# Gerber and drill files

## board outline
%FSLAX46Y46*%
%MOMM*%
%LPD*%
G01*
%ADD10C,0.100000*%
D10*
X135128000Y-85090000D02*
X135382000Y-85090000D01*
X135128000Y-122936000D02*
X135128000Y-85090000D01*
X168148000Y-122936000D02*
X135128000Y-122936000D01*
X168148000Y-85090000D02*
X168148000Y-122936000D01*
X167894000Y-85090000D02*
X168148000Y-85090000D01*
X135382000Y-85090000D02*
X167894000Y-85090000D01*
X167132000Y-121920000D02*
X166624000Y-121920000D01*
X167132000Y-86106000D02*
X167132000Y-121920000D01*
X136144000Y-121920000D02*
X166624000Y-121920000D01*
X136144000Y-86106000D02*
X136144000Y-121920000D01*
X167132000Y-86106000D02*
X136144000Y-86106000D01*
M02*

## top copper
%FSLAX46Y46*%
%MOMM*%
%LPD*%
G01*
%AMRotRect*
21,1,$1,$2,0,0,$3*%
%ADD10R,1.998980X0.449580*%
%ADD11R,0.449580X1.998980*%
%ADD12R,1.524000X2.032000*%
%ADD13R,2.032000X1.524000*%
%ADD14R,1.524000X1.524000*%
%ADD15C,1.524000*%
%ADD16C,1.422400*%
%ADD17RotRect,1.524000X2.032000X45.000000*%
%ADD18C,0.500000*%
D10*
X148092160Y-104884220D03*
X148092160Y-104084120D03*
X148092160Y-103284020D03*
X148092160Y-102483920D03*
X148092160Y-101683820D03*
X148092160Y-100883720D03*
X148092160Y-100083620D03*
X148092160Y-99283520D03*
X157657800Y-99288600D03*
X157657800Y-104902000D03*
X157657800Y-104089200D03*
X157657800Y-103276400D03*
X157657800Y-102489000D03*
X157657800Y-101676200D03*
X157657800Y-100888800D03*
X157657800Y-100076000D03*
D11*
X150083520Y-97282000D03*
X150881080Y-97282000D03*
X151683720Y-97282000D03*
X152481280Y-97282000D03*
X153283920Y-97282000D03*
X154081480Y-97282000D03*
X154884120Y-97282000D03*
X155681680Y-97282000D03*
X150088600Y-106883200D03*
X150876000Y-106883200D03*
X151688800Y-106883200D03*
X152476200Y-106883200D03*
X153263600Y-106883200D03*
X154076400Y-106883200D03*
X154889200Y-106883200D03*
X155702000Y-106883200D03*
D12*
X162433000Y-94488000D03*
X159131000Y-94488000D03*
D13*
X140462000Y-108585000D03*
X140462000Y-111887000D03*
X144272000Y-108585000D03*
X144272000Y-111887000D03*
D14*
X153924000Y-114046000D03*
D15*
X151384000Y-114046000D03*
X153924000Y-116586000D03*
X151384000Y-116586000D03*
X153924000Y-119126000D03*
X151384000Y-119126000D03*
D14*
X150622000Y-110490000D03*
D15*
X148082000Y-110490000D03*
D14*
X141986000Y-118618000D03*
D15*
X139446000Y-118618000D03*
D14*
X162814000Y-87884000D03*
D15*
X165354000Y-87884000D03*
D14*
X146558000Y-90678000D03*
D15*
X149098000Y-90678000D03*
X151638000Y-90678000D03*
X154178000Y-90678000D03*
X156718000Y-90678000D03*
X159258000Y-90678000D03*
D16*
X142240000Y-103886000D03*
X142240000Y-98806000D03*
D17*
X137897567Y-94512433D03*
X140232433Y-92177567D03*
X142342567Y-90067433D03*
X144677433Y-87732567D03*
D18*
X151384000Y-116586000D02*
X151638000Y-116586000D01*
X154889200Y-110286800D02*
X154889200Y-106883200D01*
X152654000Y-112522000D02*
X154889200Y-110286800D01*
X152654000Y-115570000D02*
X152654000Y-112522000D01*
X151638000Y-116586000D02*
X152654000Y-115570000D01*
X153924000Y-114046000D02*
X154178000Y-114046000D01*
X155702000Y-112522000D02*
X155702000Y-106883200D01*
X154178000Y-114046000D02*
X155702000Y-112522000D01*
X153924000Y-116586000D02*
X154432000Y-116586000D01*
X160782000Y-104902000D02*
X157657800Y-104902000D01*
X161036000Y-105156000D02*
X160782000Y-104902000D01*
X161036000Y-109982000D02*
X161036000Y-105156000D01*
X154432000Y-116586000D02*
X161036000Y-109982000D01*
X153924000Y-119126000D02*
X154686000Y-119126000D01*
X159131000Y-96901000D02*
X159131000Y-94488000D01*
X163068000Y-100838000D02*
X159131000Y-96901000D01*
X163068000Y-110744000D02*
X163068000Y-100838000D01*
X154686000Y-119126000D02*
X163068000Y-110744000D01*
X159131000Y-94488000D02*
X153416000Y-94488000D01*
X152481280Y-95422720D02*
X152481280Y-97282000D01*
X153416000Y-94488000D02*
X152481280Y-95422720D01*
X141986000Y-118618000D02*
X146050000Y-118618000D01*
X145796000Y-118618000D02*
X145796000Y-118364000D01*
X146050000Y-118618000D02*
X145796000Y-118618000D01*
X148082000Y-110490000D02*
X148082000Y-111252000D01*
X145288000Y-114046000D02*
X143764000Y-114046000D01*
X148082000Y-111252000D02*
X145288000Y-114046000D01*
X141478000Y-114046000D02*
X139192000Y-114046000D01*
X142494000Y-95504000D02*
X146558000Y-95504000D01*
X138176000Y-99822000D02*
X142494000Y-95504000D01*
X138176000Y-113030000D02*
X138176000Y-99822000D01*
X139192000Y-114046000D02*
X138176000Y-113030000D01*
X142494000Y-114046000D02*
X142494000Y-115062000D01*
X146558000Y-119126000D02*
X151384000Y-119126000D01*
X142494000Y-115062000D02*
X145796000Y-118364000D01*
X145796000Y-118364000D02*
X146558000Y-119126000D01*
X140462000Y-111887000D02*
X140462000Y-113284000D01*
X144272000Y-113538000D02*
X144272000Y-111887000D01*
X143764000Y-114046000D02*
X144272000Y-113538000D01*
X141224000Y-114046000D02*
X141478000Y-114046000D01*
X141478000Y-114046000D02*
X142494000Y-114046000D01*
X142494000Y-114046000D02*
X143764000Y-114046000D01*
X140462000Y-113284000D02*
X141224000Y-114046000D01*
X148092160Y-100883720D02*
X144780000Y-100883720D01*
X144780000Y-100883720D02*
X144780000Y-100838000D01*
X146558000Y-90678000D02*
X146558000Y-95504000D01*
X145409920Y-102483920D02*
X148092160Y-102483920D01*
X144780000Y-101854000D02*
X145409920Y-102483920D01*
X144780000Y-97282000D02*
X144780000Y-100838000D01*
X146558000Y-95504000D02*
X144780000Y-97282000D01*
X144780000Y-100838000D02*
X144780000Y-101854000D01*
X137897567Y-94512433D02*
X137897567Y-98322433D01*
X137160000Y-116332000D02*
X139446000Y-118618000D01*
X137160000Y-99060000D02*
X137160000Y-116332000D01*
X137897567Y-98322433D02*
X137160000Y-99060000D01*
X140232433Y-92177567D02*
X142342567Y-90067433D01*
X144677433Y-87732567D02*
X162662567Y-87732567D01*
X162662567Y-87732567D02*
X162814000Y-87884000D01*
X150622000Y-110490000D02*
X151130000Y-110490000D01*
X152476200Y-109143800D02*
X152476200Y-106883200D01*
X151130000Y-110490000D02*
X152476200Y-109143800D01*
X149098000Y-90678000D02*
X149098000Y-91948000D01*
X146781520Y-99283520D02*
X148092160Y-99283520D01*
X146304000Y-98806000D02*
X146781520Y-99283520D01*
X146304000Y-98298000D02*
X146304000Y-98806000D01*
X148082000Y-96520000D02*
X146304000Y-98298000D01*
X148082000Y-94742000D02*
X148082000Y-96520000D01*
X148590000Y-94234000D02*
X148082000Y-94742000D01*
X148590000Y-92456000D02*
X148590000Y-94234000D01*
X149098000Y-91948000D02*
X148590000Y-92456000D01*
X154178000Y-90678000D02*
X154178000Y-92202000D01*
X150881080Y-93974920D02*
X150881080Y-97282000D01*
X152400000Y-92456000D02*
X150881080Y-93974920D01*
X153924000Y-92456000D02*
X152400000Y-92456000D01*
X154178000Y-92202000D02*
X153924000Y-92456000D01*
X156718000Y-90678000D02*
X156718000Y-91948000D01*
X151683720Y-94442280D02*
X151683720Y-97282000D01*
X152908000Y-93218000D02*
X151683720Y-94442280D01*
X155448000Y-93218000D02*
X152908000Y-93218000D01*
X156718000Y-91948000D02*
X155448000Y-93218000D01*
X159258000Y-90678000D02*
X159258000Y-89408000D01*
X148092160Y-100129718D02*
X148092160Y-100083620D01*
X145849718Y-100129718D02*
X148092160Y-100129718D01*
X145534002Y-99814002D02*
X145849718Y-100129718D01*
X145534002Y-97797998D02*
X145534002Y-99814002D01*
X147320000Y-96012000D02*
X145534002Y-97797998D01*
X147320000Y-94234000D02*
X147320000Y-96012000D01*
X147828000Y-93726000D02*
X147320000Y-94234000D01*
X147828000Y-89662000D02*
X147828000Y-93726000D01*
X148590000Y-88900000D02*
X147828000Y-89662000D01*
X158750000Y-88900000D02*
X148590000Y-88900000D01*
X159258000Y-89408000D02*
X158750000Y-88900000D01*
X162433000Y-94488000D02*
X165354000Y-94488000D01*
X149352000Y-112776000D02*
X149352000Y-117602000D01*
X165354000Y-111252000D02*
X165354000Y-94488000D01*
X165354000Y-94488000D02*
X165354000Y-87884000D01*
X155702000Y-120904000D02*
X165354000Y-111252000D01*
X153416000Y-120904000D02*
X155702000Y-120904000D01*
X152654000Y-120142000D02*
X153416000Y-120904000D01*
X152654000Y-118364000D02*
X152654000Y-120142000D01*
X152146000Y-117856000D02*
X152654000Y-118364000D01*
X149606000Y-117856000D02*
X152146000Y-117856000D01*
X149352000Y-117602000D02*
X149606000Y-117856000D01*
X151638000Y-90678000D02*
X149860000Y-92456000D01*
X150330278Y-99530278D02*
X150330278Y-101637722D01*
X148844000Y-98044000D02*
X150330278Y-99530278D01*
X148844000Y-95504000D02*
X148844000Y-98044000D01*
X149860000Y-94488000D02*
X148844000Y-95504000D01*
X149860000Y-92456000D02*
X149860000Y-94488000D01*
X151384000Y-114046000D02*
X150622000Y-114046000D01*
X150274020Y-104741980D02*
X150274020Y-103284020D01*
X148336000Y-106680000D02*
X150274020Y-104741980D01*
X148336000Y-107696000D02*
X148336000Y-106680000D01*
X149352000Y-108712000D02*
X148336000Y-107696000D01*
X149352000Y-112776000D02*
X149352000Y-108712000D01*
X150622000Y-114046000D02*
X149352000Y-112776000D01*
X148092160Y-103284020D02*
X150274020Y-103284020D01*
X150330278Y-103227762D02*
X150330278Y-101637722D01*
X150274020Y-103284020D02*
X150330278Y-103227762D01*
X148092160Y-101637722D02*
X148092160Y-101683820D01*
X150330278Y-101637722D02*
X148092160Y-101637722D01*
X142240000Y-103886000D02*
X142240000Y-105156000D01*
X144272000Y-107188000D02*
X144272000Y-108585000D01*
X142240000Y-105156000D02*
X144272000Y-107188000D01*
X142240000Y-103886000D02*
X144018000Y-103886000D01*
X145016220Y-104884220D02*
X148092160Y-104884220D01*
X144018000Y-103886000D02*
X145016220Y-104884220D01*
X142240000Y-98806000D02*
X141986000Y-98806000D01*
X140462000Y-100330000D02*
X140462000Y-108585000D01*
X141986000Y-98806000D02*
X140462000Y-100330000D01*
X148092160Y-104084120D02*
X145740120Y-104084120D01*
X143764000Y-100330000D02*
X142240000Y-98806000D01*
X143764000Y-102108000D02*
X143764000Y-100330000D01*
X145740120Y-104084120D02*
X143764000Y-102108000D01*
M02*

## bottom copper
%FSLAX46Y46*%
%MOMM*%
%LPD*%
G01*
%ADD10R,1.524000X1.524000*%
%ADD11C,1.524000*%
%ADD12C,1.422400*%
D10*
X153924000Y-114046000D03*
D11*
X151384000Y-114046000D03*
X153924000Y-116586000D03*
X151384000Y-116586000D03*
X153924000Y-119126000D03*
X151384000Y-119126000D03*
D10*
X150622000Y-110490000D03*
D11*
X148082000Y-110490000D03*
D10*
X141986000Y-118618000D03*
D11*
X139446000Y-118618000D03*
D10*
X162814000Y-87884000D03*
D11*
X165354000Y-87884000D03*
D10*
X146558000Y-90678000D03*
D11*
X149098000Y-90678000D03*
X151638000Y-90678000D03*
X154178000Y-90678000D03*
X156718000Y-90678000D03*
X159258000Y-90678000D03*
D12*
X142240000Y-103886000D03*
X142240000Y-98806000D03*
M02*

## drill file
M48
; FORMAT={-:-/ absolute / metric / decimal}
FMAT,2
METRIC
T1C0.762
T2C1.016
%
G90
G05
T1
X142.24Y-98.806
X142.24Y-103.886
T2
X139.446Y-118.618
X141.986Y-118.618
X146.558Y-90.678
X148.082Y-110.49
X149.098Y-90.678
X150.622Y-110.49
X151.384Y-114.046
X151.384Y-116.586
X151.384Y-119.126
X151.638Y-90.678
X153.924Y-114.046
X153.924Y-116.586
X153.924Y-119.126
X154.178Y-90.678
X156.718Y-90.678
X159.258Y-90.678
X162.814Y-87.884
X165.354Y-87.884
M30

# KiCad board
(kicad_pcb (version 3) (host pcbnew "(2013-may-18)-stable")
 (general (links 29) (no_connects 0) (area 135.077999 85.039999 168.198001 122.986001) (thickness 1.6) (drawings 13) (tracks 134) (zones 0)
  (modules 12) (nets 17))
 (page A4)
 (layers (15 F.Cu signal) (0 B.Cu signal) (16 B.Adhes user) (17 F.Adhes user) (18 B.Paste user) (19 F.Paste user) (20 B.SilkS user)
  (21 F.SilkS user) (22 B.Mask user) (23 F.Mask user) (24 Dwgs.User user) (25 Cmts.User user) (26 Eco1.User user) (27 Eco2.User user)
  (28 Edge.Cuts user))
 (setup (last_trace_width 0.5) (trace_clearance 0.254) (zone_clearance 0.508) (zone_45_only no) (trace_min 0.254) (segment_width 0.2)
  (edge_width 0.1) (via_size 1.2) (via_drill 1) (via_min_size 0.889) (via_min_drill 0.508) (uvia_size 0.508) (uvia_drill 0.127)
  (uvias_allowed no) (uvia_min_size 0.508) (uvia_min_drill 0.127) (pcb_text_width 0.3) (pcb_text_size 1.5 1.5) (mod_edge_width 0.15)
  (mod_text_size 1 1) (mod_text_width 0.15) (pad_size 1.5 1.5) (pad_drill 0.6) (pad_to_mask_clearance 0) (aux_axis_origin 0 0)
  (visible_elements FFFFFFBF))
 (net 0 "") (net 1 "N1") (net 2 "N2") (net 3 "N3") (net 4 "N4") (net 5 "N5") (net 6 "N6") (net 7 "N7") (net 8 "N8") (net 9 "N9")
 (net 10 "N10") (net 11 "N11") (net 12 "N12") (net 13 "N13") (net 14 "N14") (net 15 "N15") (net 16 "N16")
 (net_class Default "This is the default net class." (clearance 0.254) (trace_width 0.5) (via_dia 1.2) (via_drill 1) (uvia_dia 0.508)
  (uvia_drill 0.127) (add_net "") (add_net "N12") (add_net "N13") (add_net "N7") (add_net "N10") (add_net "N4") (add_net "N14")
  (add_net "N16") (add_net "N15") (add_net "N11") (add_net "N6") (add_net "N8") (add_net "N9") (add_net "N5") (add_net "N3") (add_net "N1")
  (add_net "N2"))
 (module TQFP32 (layer F.Cu) (at 152.908 102.108)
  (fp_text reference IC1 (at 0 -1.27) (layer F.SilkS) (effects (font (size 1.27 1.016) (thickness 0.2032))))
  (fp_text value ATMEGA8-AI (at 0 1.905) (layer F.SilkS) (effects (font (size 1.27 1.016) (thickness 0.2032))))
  (pad 8 smd rect (at -4.81584 2.77622) (size 1.99898 0.44958) (layers F.Cu F.Paste F.Mask) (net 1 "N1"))
  (pad 7 smd rect (at -4.81584 1.97612) (size 1.99898 0.44958) (layers F.Cu F.Paste F.Mask) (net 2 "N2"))
  (pad 6 smd rect (at -4.81584 1.17602) (size 1.99898 0.44958) (layers F.Cu F.Paste F.Mask) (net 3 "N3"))
  (pad 5 smd rect (at -4.81584 0.37592) (size 1.99898 0.44958) (layers F.Cu F.Paste F.Mask) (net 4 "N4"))
  (pad 4 smd rect (at -4.81584 -0.42418) (size 1.99898 0.44958) (layers F.Cu F.Paste F.Mask) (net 3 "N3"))
  (pad 3 smd rect (at -4.81584 -1.22428) (size 1.99898 0.44958) (layers F.Cu F.Paste F.Mask) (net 4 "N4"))
  (pad 2 smd rect (at -4.81584 -2.02438) (size 1.99898 0.44958) (layers F.Cu F.Paste F.Mask) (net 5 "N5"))
  (pad 1 smd rect (at -4.81584 -2.82448) (size 1.99898 0.44958) (layers F.Cu F.Paste F.Mask) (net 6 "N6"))
  (pad 24 smd rect (at 4.7498 -2.8194) (size 1.99898 0.44958) (layers F.Cu F.Paste F.Mask))
  (pad 17 smd rect (at 4.7498 2.794) (size 1.99898 0.44958) (layers F.Cu F.Paste F.Mask) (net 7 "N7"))
  (pad 18 smd rect (at 4.7498 1.9812) (size 1.99898 0.44958) (layers F.Cu F.Paste F.Mask))
  (pad 19 smd rect (at 4.7498 1.1684) (size 1.99898 0.44958) (layers F.Cu F.Paste F.Mask))
  (pad 20 smd rect (at 4.7498 0.381) (size 1.99898 0.44958) (layers F.Cu F.Paste F.Mask))
  (pad 21 smd rect (at 4.7498 -0.4318) (size 1.99898 0.44958) (layers F.Cu F.Paste F.Mask))
  (pad 22 smd rect (at 4.7498 -1.2192) (size 1.99898 0.44958) (layers F.Cu F.Paste F.Mask))
  (pad 23 smd rect (at 4.7498 -2.032) (size 1.99898 0.44958) (layers F.Cu F.Paste F.Mask))
  (pad 32 smd rect (at -2.82448 -4.826) (size 0.44958 1.99898) (layers F.Cu F.Paste F.Mask))
  (pad 31 smd rect (at -2.02692 -4.826) (size 0.44958 1.99898) (layers F.Cu F.Paste F.Mask) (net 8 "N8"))
  (pad 30 smd rect (at -1.22428 -4.826) (size 0.44958 1.99898) (layers F.Cu F.Paste F.Mask) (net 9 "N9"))
  (pad 29 smd rect (at -0.42672 -4.826) (size 0.44958 1.99898) (layers F.Cu F.Paste F.Mask) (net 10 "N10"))
  (pad 28 smd rect (at 0.37592 -4.826) (size 0.44958 1.99898) (layers F.Cu F.Paste F.Mask))
  (pad 27 smd rect (at 1.17348 -4.826) (size 0.44958 1.99898) (layers F.Cu F.Paste F.Mask))
  (pad 26 smd rect (at 1.97612 -4.826) (size 0.44958 1.99898) (layers F.Cu F.Paste F.Mask))
  (pad 25 smd rect (at 2.77368 -4.826) (size 0.44958 1.99898) (layers F.Cu F.Paste F.Mask))
  (pad 9 smd rect (at -2.8194 4.7752) (size 0.44958 1.99898) (layers F.Cu F.Paste F.Mask))
  (pad 10 smd rect (at -2.032 4.7752) (size 0.44958 1.99898) (layers F.Cu F.Paste F.Mask))
  (pad 11 smd rect (at -1.2192 4.7752) (size 0.44958 1.99898) (layers F.Cu F.Paste F.Mask))
  (pad 12 smd rect (at -0.4318 4.7752) (size 0.44958 1.99898) (layers F.Cu F.Paste F.Mask) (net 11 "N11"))
  (pad 13 smd rect (at 0.3556 4.7752) (size 0.44958 1.99898) (layers F.Cu F.Paste F.Mask))
  (pad 14 smd rect (at 1.1684 4.7752) (size 0.44958 1.99898) (layers F.Cu F.Paste F.Mask))
  (pad 15 smd rect (at 1.9812 4.7752) (size 0.44958 1.99898) (layers F.Cu F.Paste F.Mask) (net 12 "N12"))
  (pad 16 smd rect (at 2.794 4.7752) (size 0.44958 1.99898) (layers F.Cu F.Paste F.Mask) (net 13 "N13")))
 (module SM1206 (layer F.Cu) (at 160.782 94.488 180)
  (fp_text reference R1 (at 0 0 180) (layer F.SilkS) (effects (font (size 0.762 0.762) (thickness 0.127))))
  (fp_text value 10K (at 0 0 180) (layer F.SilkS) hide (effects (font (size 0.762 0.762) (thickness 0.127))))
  (pad 1 smd rect (at -1.651 0 180) (size 1.524 2.032) (layers F.Cu F.Paste F.Mask) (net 3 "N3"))
  (pad 2 smd rect (at 1.651 0 180) (size 1.524 2.032) (layers F.Cu F.Paste F.Mask) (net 10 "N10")))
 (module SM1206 (layer F.Cu) (at 140.462 110.236 270)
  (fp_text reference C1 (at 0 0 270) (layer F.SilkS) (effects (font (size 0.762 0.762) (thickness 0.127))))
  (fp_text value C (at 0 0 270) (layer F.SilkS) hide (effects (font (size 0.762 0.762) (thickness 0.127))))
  (pad 1 smd rect (at -1.651 0 270) (size 1.524 2.032) (layers F.Cu F.Paste F.Mask) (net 2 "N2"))
  (pad 2 smd rect (at 1.651 0 270) (size 1.524 2.032) (layers F.Cu F.Paste F.Mask) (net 4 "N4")))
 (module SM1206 (layer F.Cu) (at 144.272 110.236 270)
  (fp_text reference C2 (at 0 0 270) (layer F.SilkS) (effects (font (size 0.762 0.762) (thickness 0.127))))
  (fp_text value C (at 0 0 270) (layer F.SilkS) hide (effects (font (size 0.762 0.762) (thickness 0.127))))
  (pad 1 smd rect (at -1.651 0 270) (size 1.524 2.032) (layers F.Cu F.Paste F.Mask) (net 1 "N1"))
  (pad 2 smd rect (at 1.651 0 270) (size 1.524 2.032) (layers F.Cu F.Paste F.Mask) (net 4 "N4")))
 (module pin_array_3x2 (layer B.Cu) (at 152.654 116.586 270)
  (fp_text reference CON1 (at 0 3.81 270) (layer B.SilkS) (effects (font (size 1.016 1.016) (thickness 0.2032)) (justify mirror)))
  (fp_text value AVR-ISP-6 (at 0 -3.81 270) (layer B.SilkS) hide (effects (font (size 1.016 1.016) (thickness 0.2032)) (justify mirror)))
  (pad 1 thru_hole rect (at -2.54 -1.27 270) (size 1.524 1.524) (drill 1.016) (layers *.Cu *.Mask B.SilkS) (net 13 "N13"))
  (pad 2 thru_hole circle (at -2.54 1.27 270) (size 1.524 1.524) (drill 1.016) (layers *.Cu *.Mask B.SilkS) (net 3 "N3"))
  (pad 3 thru_hole circle (at 0 -1.27 270) (size 1.524 1.524) (drill 1.016) (layers *.Cu *.Mask B.SilkS) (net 7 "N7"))
  (pad 4 thru_hole circle (at 0 1.27 270) (size 1.524 1.524) (drill 1.016) (layers *.Cu *.Mask B.SilkS) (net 12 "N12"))
  (pad 5 thru_hole circle (at 2.54 -1.27 270) (size 1.524 1.524) (drill 1.016) (layers *.Cu *.Mask B.SilkS) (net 10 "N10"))
  (pad 6 thru_hole circle (at 2.54 1.27 270) (size 1.524 1.524) (drill 1.016) (layers *.Cu *.Mask B.SilkS) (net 4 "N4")))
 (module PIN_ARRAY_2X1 (layer F.Cu) (at 149.352 110.49 180)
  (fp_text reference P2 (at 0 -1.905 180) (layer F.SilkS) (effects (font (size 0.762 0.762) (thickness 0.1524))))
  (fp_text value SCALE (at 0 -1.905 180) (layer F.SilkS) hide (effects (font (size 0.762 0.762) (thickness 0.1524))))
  (pad 1 thru_hole rect (at -1.27 0 180) (size 1.524 1.524) (drill 1.016) (layers *.Cu *.Mask F.SilkS) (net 11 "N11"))
  (pad 2 thru_hole circle (at 1.27 0 180) (size 1.524 1.524) (drill 1.016) (layers *.Cu *.Mask F.SilkS) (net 4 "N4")))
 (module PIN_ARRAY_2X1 (layer F.Cu) (at 140.716 118.618 180)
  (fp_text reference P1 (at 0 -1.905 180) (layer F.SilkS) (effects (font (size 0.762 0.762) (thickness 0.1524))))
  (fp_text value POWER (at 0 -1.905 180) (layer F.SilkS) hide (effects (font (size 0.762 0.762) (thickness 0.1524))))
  (pad 1 thru_hole rect (at -1.27 0 180) (size 1.524 1.524) (drill 1.016) (layers *.Cu *.Mask F.SilkS) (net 4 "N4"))
  (pad 2 thru_hole circle (at 1.27 0 180) (size 1.524 1.524) (drill 1.016) (layers *.Cu *.Mask F.SilkS) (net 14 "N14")))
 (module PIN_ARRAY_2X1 (layer F.Cu) (at 164.084 87.884)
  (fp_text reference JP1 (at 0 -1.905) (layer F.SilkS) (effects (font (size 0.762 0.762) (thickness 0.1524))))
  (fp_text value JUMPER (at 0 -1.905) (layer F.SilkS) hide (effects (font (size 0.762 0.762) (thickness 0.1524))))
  (pad 1 thru_hole rect (at -1.27 0) (size 1.524 1.524) (drill 1.016) (layers *.Cu *.Mask F.SilkS) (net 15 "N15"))
  (pad 2 thru_hole circle (at 1.27 0) (size 1.524 1.524) (drill 1.016) (layers *.Cu *.Mask F.SilkS) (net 3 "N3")))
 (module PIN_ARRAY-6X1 (layer F.Cu) (at 152.908 90.678)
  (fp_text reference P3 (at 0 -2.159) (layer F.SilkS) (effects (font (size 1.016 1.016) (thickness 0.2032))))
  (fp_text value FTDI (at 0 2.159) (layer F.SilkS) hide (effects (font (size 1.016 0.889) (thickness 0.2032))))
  (pad 1 thru_hole rect (at -6.35 0) (size 1.524 1.524) (drill 1.016) (layers *.Cu *.Mask F.SilkS) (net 4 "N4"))
  (pad 2 thru_hole circle (at -3.81 0) (size 1.524 1.524) (drill 1.016) (layers *.Cu *.Mask F.SilkS) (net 6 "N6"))
  (pad 3 thru_hole circle (at -1.27 0) (size 1.524 1.524) (drill 1.016) (layers *.Cu *.Mask F.SilkS) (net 3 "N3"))
  (pad 4 thru_hole circle (at 1.27 0) (size 1.524 1.524) (drill 1.016) (layers *.Cu *.Mask F.SilkS) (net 8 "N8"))
  (pad 5 thru_hole circle (at 3.81 0) (size 1.524 1.524) (drill 1.016) (layers *.Cu *.Mask F.SilkS) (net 9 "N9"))
  (pad 6 thru_hole circle (at 6.35 0) (size 1.524 1.524) (drill 1.016) (layers *.Cu *.Mask F.SilkS) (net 5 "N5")))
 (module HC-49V (layer F.Cu) (at 142.24 101.346 90) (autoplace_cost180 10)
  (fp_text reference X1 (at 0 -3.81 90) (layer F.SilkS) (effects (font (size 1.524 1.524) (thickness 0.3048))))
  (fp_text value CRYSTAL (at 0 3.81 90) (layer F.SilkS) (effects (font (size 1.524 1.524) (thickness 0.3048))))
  (pad 1 thru_hole circle (at -2.54 0 90) (size 1.4224 1.4224) (drill 0.762) (layers *.Cu *.Mask F.SilkS) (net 1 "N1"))
  (pad 2 thru_hole circle (at 2.54 0 90) (size 1.4224 1.4224) (drill 0.762) (layers *.Cu *.Mask F.SilkS) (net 2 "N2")))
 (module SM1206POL (layer F.Cu) (at 139.065 93.345 45)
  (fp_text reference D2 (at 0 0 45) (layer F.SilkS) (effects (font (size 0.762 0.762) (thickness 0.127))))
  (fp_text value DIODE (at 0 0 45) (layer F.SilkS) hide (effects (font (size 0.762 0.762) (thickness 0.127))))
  (pad 1 smd rect (at -1.651 0 45) (size 1.524 2.032) (layers F.Cu F.Paste F.Mask) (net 14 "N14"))
  (pad 2 smd rect (at 1.651 0 45) (size 1.524 2.032) (layers F.Cu F.Paste F.Mask) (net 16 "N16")))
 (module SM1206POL (layer F.Cu) (at 143.51 88.9 45)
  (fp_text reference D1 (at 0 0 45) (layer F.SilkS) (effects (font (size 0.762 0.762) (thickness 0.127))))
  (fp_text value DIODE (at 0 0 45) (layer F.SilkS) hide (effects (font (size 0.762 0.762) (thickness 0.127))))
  (pad 1 smd rect (at -1.651 0 45) (size 1.524 2.032) (layers F.Cu F.Paste F.Mask) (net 16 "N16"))
  (pad 2 smd rect (at 1.651 0 45) (size 1.524 2.032) (layers F.Cu F.Paste F.Mask) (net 15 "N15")))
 (gr_line (start 135.128 85.09) (end 135.382 85.09) (angle 90) (layer Edge.Cuts) (width 0.1))
 (gr_line (start 135.128 122.936) (end 135.128 85.09) (angle 90) (layer Edge.Cuts) (width 0.1))
 (gr_line (start 168.148 122.936) (end 135.128 122.936) (angle 90) (layer Edge.Cuts) (width 0.1))
 (gr_line (start 168.148 85.09) (end 168.148 122.936) (angle 90) (layer Edge.Cuts) (width 0.1))
 (gr_line (start 167.894 85.09) (end 168.148 85.09) (angle 90) (layer Edge.Cuts) (width 0.1))
 (gr_line (start 135.382 85.09) (end 167.894 85.09) (angle 90) (layer Edge.Cuts) (width 0.1))
 (gr_line (start 167.132 121.92) (end 166.624 121.92) (angle 90) (layer Edge.Cuts) (width 0.1))
 (gr_line (start 167.132 86.106) (end 167.132 121.92) (angle 90) (layer Edge.Cuts) (width 0.1))
 (gr_line (start 136.144 121.92) (end 166.624 121.92) (angle 90) (layer Edge.Cuts) (width 0.1))
 (gr_line (start 136.144 86.106) (end 136.144 121.92) (angle 90) (layer Edge.Cuts) (width 0.1))
 (gr_line (start 167.132 86.106) (end 136.144 86.106) (angle 90) (layer Edge.Cuts) (width 0.1))
 (segment (start 151.384 116.586) (end 151.638 116.586) (width 0.5) (layer F.Cu) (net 12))
 (segment (start 154.8892 110.2868) (end 154.8892 106.8832) (width 0.5) (layer F.Cu) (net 12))
 (segment (start 152.654 112.522) (end 154.8892 110.2868) (width 0.5) (layer F.Cu) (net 12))
 (segment (start 152.654 115.57) (end 152.654 112.522) (width 0.5) (layer F.Cu) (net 12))
 (segment (start 151.638 116.586) (end 152.654 115.57) (width 0.5) (layer F.Cu) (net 12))
 (segment (start 153.924 114.046) (end 154.178 114.046) (width 0.5) (layer F.Cu) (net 13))
 (segment (start 155.702 112.522) (end 155.702 106.8832) (width 0.5) (layer F.Cu) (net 13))
 (segment (start 154.178 114.046) (end 155.702 112.522) (width 0.5) (layer F.Cu) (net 13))
 (segment (start 153.924 116.586) (end 154.432 116.586) (width 0.5) (layer F.Cu) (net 7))
 (segment (start 160.782 104.902) (end 157.6578 104.902) (width 0.5) (layer F.Cu) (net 7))
 (segment (start 161.036 105.156) (end 160.782 104.902) (width 0.5) (layer F.Cu) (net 7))
 (segment (start 161.036 109.982) (end 161.036 105.156) (width 0.5) (layer F.Cu) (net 7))
 (segment (start 154.432 116.586) (end 161.036 109.982) (width 0.5) (layer F.Cu) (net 7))
 (segment (start 153.924 119.126) (end 154.686 119.126) (width 0.5) (layer F.Cu) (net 10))
 (segment (start 159.131 96.901) (end 159.131 94.488) (width 0.5) (layer F.Cu) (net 10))
 (segment (start 163.068 100.838) (end 159.131 96.901) (width 0.5) (layer F.Cu) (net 10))
 (segment (start 163.068 110.744) (end 163.068 100.838) (width 0.5) (layer F.Cu) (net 10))
 (segment (start 154.686 119.126) (end 163.068 110.744) (width 0.5) (layer F.Cu) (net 10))
 (segment (start 159.131 94.488) (end 153.416 94.488) (width 0.5) (layer F.Cu) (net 10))
 (segment (start 152.48128 95.42272) (end 152.48128 97.282) (width 0.5) (layer F.Cu) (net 10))
 (segment (start 153.416 94.488) (end 152.48128 95.42272) (width 0.5) (layer F.Cu) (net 10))
 (segment (start 141.986 118.618) (end 146.05 118.618) (width 0.5) (layer F.Cu) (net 4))
 (segment (start 145.796 118.618) (end 145.796 118.364) (width 0.5) (layer F.Cu) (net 4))
 (segment (start 146.05 118.618) (end 145.796 118.618) (width 0.5) (layer F.Cu) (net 4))
 (segment (start 148.082 110.49) (end 148.082 111.252) (width 0.5) (layer F.Cu) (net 4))
 (segment (start 145.288 114.046) (end 143.764 114.046) (width 0.5) (layer F.Cu) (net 4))
 (segment (start 148.082 111.252) (end 145.288 114.046) (width 0.5) (layer F.Cu) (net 4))
 (segment (start 141.478 114.046) (end 139.192 114.046) (width 0.5) (layer F.Cu) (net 4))
 (segment (start 142.494 95.504) (end 146.558 95.504) (width 0.5) (layer F.Cu) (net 4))
 (segment (start 138.176 99.822) (end 142.494 95.504) (width 0.5) (layer F.Cu) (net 4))
 (segment (start 138.176 113.03) (end 138.176 99.822) (width 0.5) (layer F.Cu) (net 4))
 (segment (start 139.192 114.046) (end 138.176 113.03) (width 0.5) (layer F.Cu) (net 4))
 (segment (start 142.494 114.046) (end 142.494 115.062) (width 0.5) (layer F.Cu) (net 4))
 (segment (start 146.558 119.126) (end 151.384 119.126) (width 0.5) (layer F.Cu) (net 4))
 (segment (start 142.494 115.062) (end 145.796 118.364) (width 0.5) (layer F.Cu) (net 4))
 (segment (start 145.796 118.364) (end 146.558 119.126) (width 0.5) (layer F.Cu) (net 4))
 (segment (start 140.462 111.887) (end 140.462 113.284) (width 0.5) (layer F.Cu) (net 4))
 (segment (start 144.272 113.538) (end 144.272 111.887) (width 0.5) (layer F.Cu) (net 4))
 (segment (start 143.764 114.046) (end 144.272 113.538) (width 0.5) (layer F.Cu) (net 4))
 (segment (start 141.224 114.046) (end 141.478 114.046) (width 0.5) (layer F.Cu) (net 4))
 (segment (start 141.478 114.046) (end 142.494 114.046) (width 0.5) (layer F.Cu) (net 4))
 (segment (start 142.494 114.046) (end 143.764 114.046) (width 0.5) (layer F.Cu) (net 4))
 (segment (start 140.462 113.284) (end 141.224 114.046) (width 0.5) (layer F.Cu) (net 4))
 (segment (start 148.09216 100.88372) (end 144.78 100.88372) (width 0.5) (layer F.Cu) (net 4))
 (segment (start 144.78 100.88372) (end 144.78 100.838) (width 0.5) (layer F.Cu) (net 4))
 (segment (start 146.558 90.678) (end 146.558 95.504) (width 0.5) (layer F.Cu) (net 4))
 (segment (start 145.40992 102.48392) (end 148.09216 102.48392) (width 0.5) (layer F.Cu) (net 4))
 (segment (start 144.78 101.854) (end 145.40992 102.48392) (width 0.5) (layer F.Cu) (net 4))
 (segment (start 144.78 97.282) (end 144.78 100.838) (width 0.5) (layer F.Cu) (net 4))
 (segment (start 146.558 95.504) (end 144.78 97.282) (width 0.5) (layer F.Cu) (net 4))
 (segment (start 144.78 100.838) (end 144.78 101.854) (width 0.5) (layer F.Cu) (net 4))
 (segment (start 137.897567 94.512433) (end 137.897567 98.322433) (width 0.5) (layer F.Cu) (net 14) (status 400000))
 (segment (start 137.16 116.332) (end 139.446 118.618) (width 0.5) (layer F.Cu) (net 14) (status 800000))
 (segment (start 137.16 99.06) (end 137.16 116.332) (width 0.5) (layer F.Cu) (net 14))
 (segment (start 137.897567 98.322433) (end 137.16 99.06) (width 0.5) (layer F.Cu) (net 14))
 (segment (start 140.232433 92.177567) (end 142.342567 90.067433) (width 0.5) (layer F.Cu) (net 16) (status C00000))
 (segment (start 144.677433 87.732567) (end 162.662567 87.732567) (width 0.5) (layer F.Cu) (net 15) (status C00000))
 (segment (start 162.662567 87.732567) (end 162.814 87.884) (width 0.5) (layer F.Cu) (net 15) (status C00000))
 (segment (start 150.622 110.49) (end 151.13 110.49) (width 0.5) (layer F.Cu) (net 11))
 (segment (start 152.4762 109.1438) (end 152.4762 106.8832) (width 0.5) (layer F.Cu) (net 11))
 (segment (start 151.13 110.49) (end 152.4762 109.1438) (width 0.5) (layer F.Cu) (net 11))
 (segment (start 149.098 90.678) (end 149.098 91.948) (width 0.5) (layer F.Cu) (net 6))
 (segment (start 146.78152 99.28352) (end 148.09216 99.28352) (width 0.5) (layer F.Cu) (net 6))
 (segment (start 146.304 98.806) (end 146.78152 99.28352) (width 0.5) (layer F.Cu) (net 6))
 (segment (start 146.304 98.298) (end 146.304 98.806) (width 0.5) (layer F.Cu) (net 6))
 (segment (start 148.082 96.52) (end 146.304 98.298) (width 0.5) (layer F.Cu) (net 6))
 (segment (start 148.082 94.742) (end 148.082 96.52) (width 0.5) (layer F.Cu) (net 6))
 (segment (start 148.59 94.234) (end 148.082 94.742) (width 0.5) (layer F.Cu) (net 6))
 (segment (start 148.59 92.456) (end 148.59 94.234) (width 0.5) (layer F.Cu) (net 6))
 (segment (start 149.098 91.948) (end 148.59 92.456) (width 0.5) (layer F.Cu) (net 6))
 (segment (start 154.178 90.678) (end 154.178 92.202) (width 0.5) (layer F.Cu) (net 8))
 (segment (start 150.88108 93.97492) (end 150.88108 97.282) (width 0.5) (layer F.Cu) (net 8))
 (segment (start 152.4 92.456) (end 150.88108 93.97492) (width 0.5) (layer F.Cu) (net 8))
 (segment (start 153.924 92.456) (end 152.4 92.456) (width 0.5) (layer F.Cu) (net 8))
 (segment (start 154.178 92.202) (end 153.924 92.456) (width 0.5) (layer F.Cu) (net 8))
 (segment (start 156.718 90.678) (end 156.718 91.948) (width 0.5) (layer F.Cu) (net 9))
 (segment (start 151.68372 94.44228) (end 151.68372 97.282) (width 0.5) (layer F.Cu) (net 9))
 (segment (start 152.908 93.218) (end 151.68372 94.44228) (width 0.5) (layer F.Cu) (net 9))
 (segment (start 155.448 93.218) (end 152.908 93.218) (width 0.5) (layer F.Cu) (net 9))
 (segment (start 156.718 91.948) (end 155.448 93.218) (width 0.5) (layer F.Cu) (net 9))
 (segment (start 159.258 90.678) (end 159.258 89.408) (width 0.5) (layer F.Cu) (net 5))
 (segment (start 148.09216 100.129718) (end 148.09216 100.08362) (width 0.5) (layer F.Cu) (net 5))
 (segment (start 145.849718 100.129718) (end 148.09216 100.129718) (width 0.5) (layer F.Cu) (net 5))
 (segment (start 145.534002 99.814002) (end 145.849718 100.129718) (width 0.5) (layer F.Cu) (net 5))
 (segment (start 145.534002 97.797998) (end 145.534002 99.814002) (width 0.5) (layer F.Cu) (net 5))
 (segment (start 147.32 96.012) (end 145.534002 97.797998) (width 0.5) (layer F.Cu) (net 5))
 (segment (start 147.32 94.234) (end 147.32 96.012) (width 0.5) (layer F.Cu) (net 5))
 (segment (start 147.828 93.726) (end 147.32 94.234) (width 0.5) (layer F.Cu) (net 5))
 (segment (start 147.828 89.662) (end 147.828 93.726) (width 0.5) (layer F.Cu) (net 5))
 (segment (start 148.59 88.9) (end 147.828 89.662) (width 0.5) (layer F.Cu) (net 5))
 (segment (start 158.75 88.9) (end 148.59 88.9) (width 0.5) (layer F.Cu) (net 5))
 (segment (start 159.258 89.408) (end 158.75 88.9) (width 0.5) (layer F.Cu) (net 5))
 (segment (start 162.433 94.488) (end 165.354 94.488) (width 0.5) (layer F.Cu) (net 3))
 (segment (start 149.352 112.776) (end 149.352 117.602) (width 0.5) (layer F.Cu) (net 3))
 (segment (start 165.354 111.252) (end 165.354 94.488) (width 0.5) (layer F.Cu) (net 3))
 (segment (start 165.354 94.488) (end 165.354 87.884) (width 0.5) (layer F.Cu) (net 3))
 (segment (start 155.702 120.904) (end 165.354 111.252) (width 0.5) (layer F.Cu) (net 3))
 (segment (start 153.416 120.904) (end 155.702 120.904) (width 0.5) (layer F.Cu) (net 3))
 (segment (start 152.654 120.142) (end 153.416 120.904) (width 0.5) (layer F.Cu) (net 3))
 (segment (start 152.654 118.364) (end 152.654 120.142) (width 0.5) (layer F.Cu) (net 3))
 (segment (start 152.146 117.856) (end 152.654 118.364) (width 0.5) (layer F.Cu) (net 3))
 (segment (start 149.606 117.856) (end 152.146 117.856) (width 0.5) (layer F.Cu) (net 3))
 (segment (start 149.352 117.602) (end 149.606 117.856) (width 0.5) (layer F.Cu) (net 3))
 (segment (start 151.638 90.678) (end 149.86 92.456) (width 0.5) (layer F.Cu) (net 3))
 (segment (start 150.330278 99.530278) (end 150.330278 101.637722) (width 0.5) (layer F.Cu) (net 3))
 (segment (start 148.844 98.044) (end 150.330278 99.530278) (width 0.5) (layer F.Cu) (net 3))
 (segment (start 148.844 95.504) (end 148.844 98.044) (width 0.5) (layer F.Cu) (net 3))
 (segment (start 149.86 94.488) (end 148.844 95.504) (width 0.5) (layer F.Cu) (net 3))
 (segment (start 149.86 92.456) (end 149.86 94.488) (width 0.5) (layer F.Cu) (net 3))
 (segment (start 151.384 114.046) (end 150.622 114.046) (width 0.5) (layer F.Cu) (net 3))
 (segment (start 150.27402 104.74198) (end 150.27402 103.28402) (width 0.5) (layer F.Cu) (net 3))
 (segment (start 148.336 106.68) (end 150.27402 104.74198) (width 0.5) (layer F.Cu) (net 3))
 (segment (start 148.336 107.696) (end 148.336 106.68) (width 0.5) (layer F.Cu) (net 3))
 (segment (start 149.352 108.712) (end 148.336 107.696) (width 0.5) (layer F.Cu) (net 3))
 (segment (start 149.352 112.776) (end 149.352 108.712) (width 0.5) (layer F.Cu) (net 3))
 (segment (start 150.622 114.046) (end 149.352 112.776) (width 0.5) (layer F.Cu) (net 3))
 (segment (start 148.09216 103.28402) (end 150.27402 103.28402) (width 0.5) (layer F.Cu) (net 3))
 (segment (start 150.330278 103.227762) (end 150.330278 101.637722) (width 0.5) (layer F.Cu) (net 3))
 (segment (start 150.27402 103.28402) (end 150.330278 103.227762) (width 0.5) (layer F.Cu) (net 3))
 (segment (start 148.09216 101.637722) (end 148.09216 101.68382) (width 0.5) (layer F.Cu) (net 3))
 (segment (start 150.330278 101.637722) (end 148.09216 101.637722) (width 0.5) (layer F.Cu) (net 3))
 (segment (start 142.24 103.886) (end 142.24 105.156) (width 0.5) (layer F.Cu) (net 1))
 (segment (start 144.272 107.188) (end 144.272 108.585) (width 0.5) (layer F.Cu) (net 1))
 (segment (start 142.24 105.156) (end 144.272 107.188) (width 0.5) (layer F.Cu) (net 1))
 (segment (start 142.24 103.886) (end 144.018 103.886) (width 0.5) (layer F.Cu) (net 1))
 (segment (start 145.01622 104.88422) (end 148.09216 104.88422) (width 0.5) (layer F.Cu) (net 1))
 (segment (start 144.018 103.886) (end 145.01622 104.88422) (width 0.5) (layer F.Cu) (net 1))
 (segment (start 142.24 98.806) (end 141.986 98.806) (width 0.5) (layer F.Cu) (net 2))
 (segment (start 140.462 100.33) (end 140.462 108.585) (width 0.5) (layer F.Cu) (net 2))
 (segment (start 141.986 98.806) (end 140.462 100.33) (width 0.5) (layer F.Cu) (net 2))
 (segment (start 148.09216 104.08412) (end 145.74012 104.08412) (width 0.5) (layer F.Cu) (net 2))
 (segment (start 143.764 100.33) (end 142.24 98.806) (width 0.5) (layer F.Cu) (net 2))
 (segment (start 143.764 102.108) (end 143.764 100.33) (width 0.5) (layer F.Cu) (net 2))
 (segment (start 145.74012 104.08412) (end 143.764 102.108) (width 0.5) (layer F.Cu) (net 2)))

